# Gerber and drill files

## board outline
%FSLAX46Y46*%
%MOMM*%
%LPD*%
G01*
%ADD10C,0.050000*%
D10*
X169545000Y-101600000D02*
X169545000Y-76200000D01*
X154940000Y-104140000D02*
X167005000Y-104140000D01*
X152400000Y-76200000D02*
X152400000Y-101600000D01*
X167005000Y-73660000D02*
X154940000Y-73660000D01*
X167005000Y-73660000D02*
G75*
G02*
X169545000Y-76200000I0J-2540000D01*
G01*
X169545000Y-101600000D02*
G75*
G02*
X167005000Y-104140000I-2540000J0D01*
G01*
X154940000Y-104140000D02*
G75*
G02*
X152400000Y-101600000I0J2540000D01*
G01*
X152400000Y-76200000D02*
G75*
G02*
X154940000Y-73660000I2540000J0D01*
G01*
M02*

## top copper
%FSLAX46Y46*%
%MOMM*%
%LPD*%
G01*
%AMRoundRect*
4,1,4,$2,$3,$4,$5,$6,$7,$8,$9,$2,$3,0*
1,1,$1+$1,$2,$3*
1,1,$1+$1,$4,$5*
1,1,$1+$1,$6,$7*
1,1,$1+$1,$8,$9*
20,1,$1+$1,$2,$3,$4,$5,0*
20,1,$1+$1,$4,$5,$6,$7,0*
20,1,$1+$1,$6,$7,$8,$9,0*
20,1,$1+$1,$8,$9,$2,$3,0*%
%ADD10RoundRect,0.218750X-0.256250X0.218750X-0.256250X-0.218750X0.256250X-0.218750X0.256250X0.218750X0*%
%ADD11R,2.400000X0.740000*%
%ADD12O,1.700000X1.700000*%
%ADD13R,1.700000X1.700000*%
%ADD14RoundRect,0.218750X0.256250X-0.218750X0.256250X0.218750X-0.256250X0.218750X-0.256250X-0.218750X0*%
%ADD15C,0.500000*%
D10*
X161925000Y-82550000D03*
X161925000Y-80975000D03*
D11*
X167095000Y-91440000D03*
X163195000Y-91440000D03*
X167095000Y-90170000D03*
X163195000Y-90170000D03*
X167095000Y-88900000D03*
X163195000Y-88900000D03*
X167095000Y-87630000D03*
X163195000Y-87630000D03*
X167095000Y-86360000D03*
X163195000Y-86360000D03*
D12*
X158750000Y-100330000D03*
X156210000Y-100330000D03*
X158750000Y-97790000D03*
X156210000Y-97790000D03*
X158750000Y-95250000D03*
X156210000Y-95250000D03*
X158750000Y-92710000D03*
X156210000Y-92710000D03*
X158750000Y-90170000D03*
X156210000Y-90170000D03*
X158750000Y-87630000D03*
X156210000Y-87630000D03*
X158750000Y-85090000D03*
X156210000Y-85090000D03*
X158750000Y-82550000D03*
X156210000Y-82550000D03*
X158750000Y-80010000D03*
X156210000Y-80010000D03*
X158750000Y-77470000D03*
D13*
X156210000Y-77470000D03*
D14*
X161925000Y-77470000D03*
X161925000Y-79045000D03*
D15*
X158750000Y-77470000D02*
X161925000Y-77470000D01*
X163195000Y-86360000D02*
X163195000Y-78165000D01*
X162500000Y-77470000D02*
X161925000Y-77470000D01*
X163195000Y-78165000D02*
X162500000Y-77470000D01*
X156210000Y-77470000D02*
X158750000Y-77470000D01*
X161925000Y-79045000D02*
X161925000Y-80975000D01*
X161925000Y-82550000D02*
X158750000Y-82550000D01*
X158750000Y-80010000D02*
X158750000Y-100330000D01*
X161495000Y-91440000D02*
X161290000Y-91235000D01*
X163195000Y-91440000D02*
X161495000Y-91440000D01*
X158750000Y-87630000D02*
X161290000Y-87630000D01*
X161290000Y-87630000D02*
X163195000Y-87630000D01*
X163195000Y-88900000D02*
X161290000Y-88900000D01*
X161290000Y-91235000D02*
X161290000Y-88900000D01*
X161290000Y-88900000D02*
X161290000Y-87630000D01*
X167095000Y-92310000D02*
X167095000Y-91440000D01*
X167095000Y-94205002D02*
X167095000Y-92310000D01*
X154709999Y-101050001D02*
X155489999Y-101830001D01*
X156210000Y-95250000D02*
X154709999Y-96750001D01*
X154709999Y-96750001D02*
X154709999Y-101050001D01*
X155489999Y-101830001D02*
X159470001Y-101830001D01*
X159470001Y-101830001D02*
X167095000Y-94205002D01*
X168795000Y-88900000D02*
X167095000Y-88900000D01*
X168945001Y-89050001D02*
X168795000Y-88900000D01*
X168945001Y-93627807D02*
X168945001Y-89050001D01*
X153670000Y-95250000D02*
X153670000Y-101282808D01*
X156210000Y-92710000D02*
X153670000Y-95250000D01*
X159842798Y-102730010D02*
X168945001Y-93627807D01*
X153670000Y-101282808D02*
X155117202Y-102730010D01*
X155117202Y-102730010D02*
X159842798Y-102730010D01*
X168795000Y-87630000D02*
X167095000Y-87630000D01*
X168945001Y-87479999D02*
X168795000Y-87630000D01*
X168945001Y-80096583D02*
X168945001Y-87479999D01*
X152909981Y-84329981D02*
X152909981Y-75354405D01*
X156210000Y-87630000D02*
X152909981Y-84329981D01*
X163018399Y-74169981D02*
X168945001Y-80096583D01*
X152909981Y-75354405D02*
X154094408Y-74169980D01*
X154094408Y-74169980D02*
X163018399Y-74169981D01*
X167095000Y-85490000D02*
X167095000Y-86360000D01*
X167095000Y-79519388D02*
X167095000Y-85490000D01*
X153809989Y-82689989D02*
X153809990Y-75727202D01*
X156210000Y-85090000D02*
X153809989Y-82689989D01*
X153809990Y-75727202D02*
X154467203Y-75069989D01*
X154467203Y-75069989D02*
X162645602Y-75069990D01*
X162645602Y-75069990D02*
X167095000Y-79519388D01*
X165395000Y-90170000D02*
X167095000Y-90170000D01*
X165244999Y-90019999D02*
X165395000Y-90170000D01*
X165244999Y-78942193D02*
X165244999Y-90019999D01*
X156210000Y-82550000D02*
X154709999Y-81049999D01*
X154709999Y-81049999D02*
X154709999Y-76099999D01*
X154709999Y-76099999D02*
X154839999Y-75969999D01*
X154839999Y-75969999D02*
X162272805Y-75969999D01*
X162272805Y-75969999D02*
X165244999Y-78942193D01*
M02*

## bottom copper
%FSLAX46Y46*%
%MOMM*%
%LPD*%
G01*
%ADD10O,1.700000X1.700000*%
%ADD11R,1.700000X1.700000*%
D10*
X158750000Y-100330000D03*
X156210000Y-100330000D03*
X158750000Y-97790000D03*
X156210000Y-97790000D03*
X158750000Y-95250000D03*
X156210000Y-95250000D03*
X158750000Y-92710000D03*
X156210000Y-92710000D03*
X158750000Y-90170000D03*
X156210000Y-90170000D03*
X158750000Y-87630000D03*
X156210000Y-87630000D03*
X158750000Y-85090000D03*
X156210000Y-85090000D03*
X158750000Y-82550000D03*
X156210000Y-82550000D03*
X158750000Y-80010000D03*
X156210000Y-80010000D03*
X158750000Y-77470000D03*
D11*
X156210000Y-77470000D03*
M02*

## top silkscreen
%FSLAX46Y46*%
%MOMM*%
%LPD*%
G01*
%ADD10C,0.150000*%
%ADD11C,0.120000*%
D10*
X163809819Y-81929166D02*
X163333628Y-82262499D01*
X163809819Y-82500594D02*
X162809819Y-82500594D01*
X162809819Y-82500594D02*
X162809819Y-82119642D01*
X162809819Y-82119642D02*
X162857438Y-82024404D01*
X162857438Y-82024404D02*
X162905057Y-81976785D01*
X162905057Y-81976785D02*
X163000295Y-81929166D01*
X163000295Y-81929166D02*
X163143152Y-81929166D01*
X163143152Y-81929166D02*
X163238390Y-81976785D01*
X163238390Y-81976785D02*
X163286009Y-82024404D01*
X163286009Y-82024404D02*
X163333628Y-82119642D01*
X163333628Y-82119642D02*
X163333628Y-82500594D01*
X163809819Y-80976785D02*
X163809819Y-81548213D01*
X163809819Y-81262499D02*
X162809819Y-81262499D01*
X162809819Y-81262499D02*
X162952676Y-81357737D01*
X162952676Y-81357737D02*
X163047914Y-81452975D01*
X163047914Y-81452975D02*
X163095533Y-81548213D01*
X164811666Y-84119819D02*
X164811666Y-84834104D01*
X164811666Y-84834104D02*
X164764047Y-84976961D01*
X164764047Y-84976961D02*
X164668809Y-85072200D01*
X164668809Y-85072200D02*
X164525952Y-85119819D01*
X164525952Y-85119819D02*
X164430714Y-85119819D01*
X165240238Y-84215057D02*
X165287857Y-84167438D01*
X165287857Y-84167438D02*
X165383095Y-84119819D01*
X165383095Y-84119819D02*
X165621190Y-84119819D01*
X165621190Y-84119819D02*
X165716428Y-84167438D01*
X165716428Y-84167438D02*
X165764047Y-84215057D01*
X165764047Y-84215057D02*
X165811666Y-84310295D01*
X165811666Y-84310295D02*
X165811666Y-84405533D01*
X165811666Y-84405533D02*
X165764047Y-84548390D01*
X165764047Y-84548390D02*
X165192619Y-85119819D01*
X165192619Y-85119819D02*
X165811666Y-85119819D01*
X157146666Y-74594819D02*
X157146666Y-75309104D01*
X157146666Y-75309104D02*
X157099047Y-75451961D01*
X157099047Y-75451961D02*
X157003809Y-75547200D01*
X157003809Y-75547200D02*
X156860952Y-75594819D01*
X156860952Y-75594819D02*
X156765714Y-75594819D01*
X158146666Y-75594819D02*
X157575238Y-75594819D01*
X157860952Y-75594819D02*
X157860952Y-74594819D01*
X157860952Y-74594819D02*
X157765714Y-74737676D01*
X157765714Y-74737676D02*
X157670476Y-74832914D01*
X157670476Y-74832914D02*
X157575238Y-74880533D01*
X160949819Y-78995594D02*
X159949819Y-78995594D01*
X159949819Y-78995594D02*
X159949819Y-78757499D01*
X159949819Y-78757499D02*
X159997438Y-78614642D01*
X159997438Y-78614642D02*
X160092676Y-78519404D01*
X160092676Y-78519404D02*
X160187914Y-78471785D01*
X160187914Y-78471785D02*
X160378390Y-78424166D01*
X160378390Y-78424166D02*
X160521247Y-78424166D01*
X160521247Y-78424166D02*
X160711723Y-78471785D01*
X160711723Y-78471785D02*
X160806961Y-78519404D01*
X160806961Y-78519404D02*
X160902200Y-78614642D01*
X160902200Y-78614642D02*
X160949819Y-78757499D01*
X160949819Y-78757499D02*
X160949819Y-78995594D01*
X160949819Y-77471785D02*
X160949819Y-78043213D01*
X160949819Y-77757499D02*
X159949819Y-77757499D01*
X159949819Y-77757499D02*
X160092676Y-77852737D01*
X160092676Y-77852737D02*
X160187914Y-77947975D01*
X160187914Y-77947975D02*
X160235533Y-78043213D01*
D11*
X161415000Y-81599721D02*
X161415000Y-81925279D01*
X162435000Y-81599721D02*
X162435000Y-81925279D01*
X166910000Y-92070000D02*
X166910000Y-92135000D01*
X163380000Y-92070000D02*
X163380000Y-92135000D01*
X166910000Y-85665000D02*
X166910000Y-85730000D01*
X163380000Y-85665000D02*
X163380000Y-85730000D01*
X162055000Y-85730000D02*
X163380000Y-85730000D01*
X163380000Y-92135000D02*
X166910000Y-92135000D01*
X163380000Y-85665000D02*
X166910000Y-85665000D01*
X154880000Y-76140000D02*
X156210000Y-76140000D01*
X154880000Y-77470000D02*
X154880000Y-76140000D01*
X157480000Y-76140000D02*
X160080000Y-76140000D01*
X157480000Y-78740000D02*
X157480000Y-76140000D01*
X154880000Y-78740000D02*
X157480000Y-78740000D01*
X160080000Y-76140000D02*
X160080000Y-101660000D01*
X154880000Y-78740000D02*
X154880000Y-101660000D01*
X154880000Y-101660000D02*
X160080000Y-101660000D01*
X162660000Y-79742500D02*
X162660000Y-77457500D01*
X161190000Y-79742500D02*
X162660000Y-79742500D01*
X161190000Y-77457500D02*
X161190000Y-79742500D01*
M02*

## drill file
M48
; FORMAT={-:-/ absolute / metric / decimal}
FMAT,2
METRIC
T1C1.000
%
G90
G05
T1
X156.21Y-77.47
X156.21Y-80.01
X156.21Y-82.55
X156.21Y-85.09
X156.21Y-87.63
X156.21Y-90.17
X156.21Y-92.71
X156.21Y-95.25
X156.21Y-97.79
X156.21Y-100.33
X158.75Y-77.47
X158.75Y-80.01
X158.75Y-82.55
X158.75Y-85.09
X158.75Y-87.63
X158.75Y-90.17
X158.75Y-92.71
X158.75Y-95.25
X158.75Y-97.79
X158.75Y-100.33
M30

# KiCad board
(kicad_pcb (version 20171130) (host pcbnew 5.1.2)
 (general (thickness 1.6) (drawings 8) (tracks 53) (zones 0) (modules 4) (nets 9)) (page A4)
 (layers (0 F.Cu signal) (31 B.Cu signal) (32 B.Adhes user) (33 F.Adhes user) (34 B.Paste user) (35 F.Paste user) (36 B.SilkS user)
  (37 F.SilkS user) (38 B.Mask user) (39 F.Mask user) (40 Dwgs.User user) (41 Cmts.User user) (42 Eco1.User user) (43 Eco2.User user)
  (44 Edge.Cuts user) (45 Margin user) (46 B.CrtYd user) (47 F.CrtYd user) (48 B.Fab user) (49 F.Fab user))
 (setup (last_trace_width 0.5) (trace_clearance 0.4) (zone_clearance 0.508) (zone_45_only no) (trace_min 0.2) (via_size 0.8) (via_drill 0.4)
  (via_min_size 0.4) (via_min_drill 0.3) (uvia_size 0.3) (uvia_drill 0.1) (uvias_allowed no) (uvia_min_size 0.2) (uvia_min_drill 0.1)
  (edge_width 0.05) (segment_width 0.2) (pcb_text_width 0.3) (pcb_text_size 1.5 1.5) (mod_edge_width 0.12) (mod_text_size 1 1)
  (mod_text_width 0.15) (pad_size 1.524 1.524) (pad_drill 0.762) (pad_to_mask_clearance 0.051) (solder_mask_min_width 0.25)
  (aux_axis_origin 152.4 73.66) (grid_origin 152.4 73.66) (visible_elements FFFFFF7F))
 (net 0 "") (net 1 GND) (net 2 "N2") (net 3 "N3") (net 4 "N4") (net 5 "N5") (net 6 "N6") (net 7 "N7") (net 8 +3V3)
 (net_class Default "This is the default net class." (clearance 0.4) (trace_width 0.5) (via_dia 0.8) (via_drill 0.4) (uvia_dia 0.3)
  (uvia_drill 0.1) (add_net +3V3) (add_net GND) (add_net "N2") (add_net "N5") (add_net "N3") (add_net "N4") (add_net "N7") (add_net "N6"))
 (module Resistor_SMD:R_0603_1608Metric (layer F.Cu) (at 161.925 81.7625 270)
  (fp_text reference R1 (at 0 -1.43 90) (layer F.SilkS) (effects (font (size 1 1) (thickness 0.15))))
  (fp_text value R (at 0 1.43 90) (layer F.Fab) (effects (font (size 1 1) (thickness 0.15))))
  (fp_line (start -0.162779 0.51) (end 0.162779 0.51) (layer F.SilkS) (width 0.12))
  (fp_line (start -0.162779 -0.51) (end 0.162779 -0.51) (layer F.SilkS) (width 0.12))
  (pad 2 smd roundrect (at 0.7875 0 270) (size 0.875 0.95) (layers F.Cu F.Paste F.Mask) (roundrect_rratio 0.25) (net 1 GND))
  (pad 1 smd roundrect (at -0.7875 0 270) (size 0.875 0.95) (layers F.Cu F.Paste F.Mask) (roundrect_rratio 0.25) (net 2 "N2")))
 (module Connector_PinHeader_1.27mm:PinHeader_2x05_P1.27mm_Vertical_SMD (layer F.Cu) (at 165.145 88.9)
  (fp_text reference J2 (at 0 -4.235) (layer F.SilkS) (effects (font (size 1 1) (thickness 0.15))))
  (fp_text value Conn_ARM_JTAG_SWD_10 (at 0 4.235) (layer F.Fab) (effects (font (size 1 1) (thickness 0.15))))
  (fp_line (start 1.765 3.17) (end 1.765 3.235) (layer F.SilkS) (width 0.12))
  (fp_line (start -1.765 3.17) (end -1.765 3.235) (layer F.SilkS) (width 0.12))
  (fp_line (start 1.765 -3.235) (end 1.765 -3.17) (layer F.SilkS) (width 0.12))
  (fp_line (start -1.765 -3.235) (end -1.765 -3.17) (layer F.SilkS) (width 0.12))
  (fp_line (start -3.09 -3.17) (end -1.765 -3.17) (layer F.SilkS) (width 0.12))
  (fp_line (start -1.765 3.235) (end 1.765 3.235) (layer F.SilkS) (width 0.12))
  (fp_line (start -1.765 -3.235) (end 1.765 -3.235) (layer F.SilkS) (width 0.12))
  (pad 10 smd rect (at 1.95 2.54) (size 2.4 0.74) (layers F.Cu F.Paste F.Mask) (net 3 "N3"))
  (pad 9 smd rect (at -1.95 2.54) (size 2.4 0.74) (layers F.Cu F.Paste F.Mask) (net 1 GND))
  (pad 8 smd rect (at 1.95 1.27) (size 2.4 0.74) (layers F.Cu F.Paste F.Mask) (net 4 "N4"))
  (pad 7 smd rect (at -1.95 1.27) (size 2.4 0.74) (layers F.Cu F.Paste F.Mask))
  (pad 6 smd rect (at 1.95 0) (size 2.4 0.74) (layers F.Cu F.Paste F.Mask) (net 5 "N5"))
  (pad 5 smd rect (at -1.95 0) (size 2.4 0.74) (layers F.Cu F.Paste F.Mask) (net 1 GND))
  (pad 4 smd rect (at 1.95 -1.27) (size 2.4 0.74) (layers F.Cu F.Paste F.Mask) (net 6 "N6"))
  (pad 3 smd rect (at -1.95 -1.27) (size 2.4 0.74) (layers F.Cu F.Paste F.Mask) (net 1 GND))
  (pad 2 smd rect (at 1.95 -2.54) (size 2.4 0.74) (layers F.Cu F.Paste F.Mask) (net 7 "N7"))
  (pad 1 smd rect (at -1.95 -2.54) (size 2.4 0.74) (layers F.Cu F.Paste F.Mask) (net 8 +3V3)))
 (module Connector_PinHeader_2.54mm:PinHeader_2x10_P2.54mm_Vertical (layer F.Cu) (at 156.21 77.47)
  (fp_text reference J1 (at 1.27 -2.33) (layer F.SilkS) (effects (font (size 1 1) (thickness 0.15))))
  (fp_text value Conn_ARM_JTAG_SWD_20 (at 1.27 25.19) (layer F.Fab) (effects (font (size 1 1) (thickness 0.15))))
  (fp_line (start -1.33 -1.33) (end 0 -1.33) (layer F.SilkS) (width 0.12))
  (fp_line (start -1.33 0) (end -1.33 -1.33) (layer F.SilkS) (width 0.12))
  (fp_line (start 1.27 -1.33) (end 3.87 -1.33) (layer F.SilkS) (width 0.12))
  (fp_line (start 1.27 1.27) (end 1.27 -1.33) (layer F.SilkS) (width 0.12))
  (fp_line (start -1.33 1.27) (end 1.27 1.27) (layer F.SilkS) (width 0.12))
  (fp_line (start 3.87 -1.33) (end 3.87 24.19) (layer F.SilkS) (width 0.12))
  (fp_line (start -1.33 1.27) (end -1.33 24.19) (layer F.SilkS) (width 0.12))
  (fp_line (start -1.33 24.19) (end 3.87 24.19) (layer F.SilkS) (width 0.12))
  (pad 20 thru_hole oval (at 2.54 22.86) (size 1.7 1.7) (drill 1) (layers *.Cu *.Mask) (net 1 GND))
  (pad 19 thru_hole oval (at 0 22.86) (size 1.7 1.7) (drill 1) (layers *.Cu *.Mask))
  (pad 18 thru_hole oval (at 2.54 20.32) (size 1.7 1.7) (drill 1) (layers *.Cu *.Mask) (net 1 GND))
  (pad 17 thru_hole oval (at 0 20.32) (size 1.7 1.7) (drill 1) (layers *.Cu *.Mask))
  (pad 16 thru_hole oval (at 2.54 17.78) (size 1.7 1.7) (drill 1) (layers *.Cu *.Mask) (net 1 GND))
  (pad 15 thru_hole oval (at 0 17.78) (size 1.7 1.7) (drill 1) (layers *.Cu *.Mask) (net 3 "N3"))
  (pad 14 thru_hole oval (at 2.54 15.24) (size 1.7 1.7) (drill 1) (layers *.Cu *.Mask) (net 1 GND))
  (pad 13 thru_hole oval (at 0 15.24) (size 1.7 1.7) (drill 1) (layers *.Cu *.Mask) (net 5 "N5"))
  (pad 12 thru_hole oval (at 2.54 12.7) (size 1.7 1.7) (drill 1) (layers *.Cu *.Mask) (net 1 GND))
  (pad 11 thru_hole oval (at 0 12.7) (size 1.7 1.7) (drill 1) (layers *.Cu *.Mask))
  (pad 10 thru_hole oval (at 2.54 10.16) (size 1.7 1.7) (drill 1) (layers *.Cu *.Mask) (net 1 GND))
  (pad 9 thru_hole oval (at 0 10.16) (size 1.7 1.7) (drill 1) (layers *.Cu *.Mask) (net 6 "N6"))
  (pad 8 thru_hole oval (at 2.54 7.62) (size 1.7 1.7) (drill 1) (layers *.Cu *.Mask) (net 1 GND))
  (pad 7 thru_hole oval (at 0 7.62) (size 1.7 1.7) (drill 1) (layers *.Cu *.Mask) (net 7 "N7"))
  (pad 6 thru_hole oval (at 2.54 5.08) (size 1.7 1.7) (drill 1) (layers *.Cu *.Mask) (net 1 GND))
  (pad 5 thru_hole oval (at 0 5.08) (size 1.7 1.7) (drill 1) (layers *.Cu *.Mask) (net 4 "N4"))
  (pad 4 thru_hole oval (at 2.54 2.54) (size 1.7 1.7) (drill 1) (layers *.Cu *.Mask) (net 1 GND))
  (pad 3 thru_hole oval (at 0 2.54) (size 1.7 1.7) (drill 1) (layers *.Cu *.Mask))
  (pad 2 thru_hole oval (at 2.54 0) (size 1.7 1.7) (drill 1) (layers *.Cu *.Mask) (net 8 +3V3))
  (pad 1 thru_hole rect (at 0 0) (size 1.7 1.7) (drill 1) (layers *.Cu *.Mask) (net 8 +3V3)))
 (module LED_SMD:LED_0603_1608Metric (layer F.Cu) (at 161.925 78.2575 90)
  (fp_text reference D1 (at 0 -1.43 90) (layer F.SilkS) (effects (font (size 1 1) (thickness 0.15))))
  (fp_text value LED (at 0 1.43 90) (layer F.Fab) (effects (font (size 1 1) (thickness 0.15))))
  (fp_line (start -1.485 0.735) (end 0.8 0.735) (layer F.SilkS) (width 0.12))
  (fp_line (start -1.485 -0.735) (end -1.485 0.735) (layer F.SilkS) (width 0.12))
  (fp_line (start 0.8 -0.735) (end -1.485 -0.735) (layer F.SilkS) (width 0.12))
  (pad 2 smd roundrect (at 0.7875 0 90) (size 0.875 0.95) (layers F.Cu F.Paste F.Mask) (roundrect_rratio 0.25) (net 8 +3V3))
  (pad 1 smd roundrect (at -0.7875 0 90) (size 0.875 0.95) (layers F.Cu F.Paste F.Mask) (roundrect_rratio 0.25) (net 2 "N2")))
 (gr_line (start 169.545 101.6) (end 169.545 76.2) (layer Edge.Cuts) (width 0.05))
 (gr_line (start 154.94 104.14) (end 167.005 104.14) (layer Edge.Cuts) (width 0.05))
 (gr_line (start 152.4 76.2) (end 152.4 101.6) (layer Edge.Cuts) (width 0.05))
 (gr_line (start 167.005 73.66) (end 154.94 73.66) (layer Edge.Cuts) (width 0.05))
 (gr_arc (start 167.005 76.2) (end 169.545 76.2) (angle -90) (layer Edge.Cuts) (width 0.05))
 (gr_arc (start 167.005 101.6) (end 167.005 104.14) (angle -90) (layer Edge.Cuts) (width 0.05))
 (gr_arc (start 154.94 101.6) (end 152.4 101.6) (angle -90) (layer Edge.Cuts) (width 0.05))
 (gr_arc (start 154.94 76.2) (end 154.94 73.66) (angle -90) (layer Edge.Cuts) (width 0.05))
 (segment (start 158.75 77.47) (end 161.925 77.47) (width 0.5) (layer F.Cu) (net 8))
 (segment (start 163.195 86.36) (end 163.195 78.165) (width 0.5) (layer F.Cu) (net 8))
 (segment (start 162.5 77.47) (end 161.925 77.47) (width 0.5) (layer F.Cu) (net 8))
 (segment (start 163.195 78.165) (end 162.5 77.47) (width 0.5) (layer F.Cu) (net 8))
 (segment (start 156.21 77.47) (end 158.75 77.47) (width 0.5) (layer F.Cu) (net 8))
 (segment (start 161.925 79.045) (end 161.925 80.975) (width 0.5) (layer F.Cu) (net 2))
 (segment (start 161.925 82.55) (end 158.75 82.55) (width 0.5) (layer F.Cu) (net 1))
 (segment (start 158.75 80.01) (end 158.75 100.33) (width 0.5) (layer F.Cu) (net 1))
 (segment (start 161.495 91.44) (end 161.29 91.235) (width 0.5) (layer F.Cu) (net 1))
 (segment (start 163.195 91.44) (end 161.495 91.44) (width 0.5) (layer F.Cu) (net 1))
 (segment (start 158.75 87.63) (end 161.29 87.63) (width 0.5) (layer F.Cu) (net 1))
 (segment (start 161.29 87.63) (end 163.195 87.63) (width 0.5) (layer F.Cu) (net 1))
 (segment (start 163.195 88.9) (end 161.29 88.9) (width 0.5) (layer F.Cu) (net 1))
 (segment (start 161.29 91.235) (end 161.29 88.9) (width 0.5) (layer F.Cu) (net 1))
 (segment (start 161.29 88.9) (end 161.29 87.63) (width 0.5) (layer F.Cu) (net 1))
 (segment (start 167.095 92.31) (end 167.095 91.44) (width 0.5) (layer F.Cu) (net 3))
 (segment (start 167.095 94.205002) (end 167.095 92.31) (width 0.5) (layer F.Cu) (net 3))
 (segment (start 154.709999 101.050001) (end 155.489999 101.830001) (width 0.5) (layer F.Cu) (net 3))
 (segment (start 156.21 95.25) (end 154.709999 96.750001) (width 0.5) (layer F.Cu) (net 3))
 (segment (start 154.709999 96.750001) (end 154.709999 101.050001) (width 0.5) (layer F.Cu) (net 3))
 (segment (start 155.489999 101.830001) (end 159.470001 101.830001) (width 0.5) (layer F.Cu) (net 3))
 (segment (start 159.470001 101.830001) (end 167.095 94.205002) (width 0.5) (layer F.Cu) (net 3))
 (segment (start 168.795 88.9) (end 167.095 88.9) (width 0.5) (layer F.Cu) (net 5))
 (segment (start 168.945001 89.050001) (end 168.795 88.9) (width 0.5) (layer F.Cu) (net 5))
 (segment (start 168.945001 93.627807) (end 168.945001 89.050001) (width 0.5) (layer F.Cu) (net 5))
 (segment (start 153.67 95.25) (end 153.67 101.282808) (width 0.5) (layer F.Cu) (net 5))
 (segment (start 156.21 92.71) (end 153.67 95.25) (width 0.5) (layer F.Cu) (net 5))
 (segment (start 159.842798 102.73001) (end 168.945001 93.627807) (width 0.5) (layer F.Cu) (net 5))
 (segment (start 153.67 101.282808) (end 155.117202 102.73001) (width 0.5) (layer F.Cu) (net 5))
 (segment (start 155.117202 102.73001) (end 159.842798 102.73001) (width 0.5) (layer F.Cu) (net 5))
 (segment (start 168.795 87.63) (end 167.095 87.63) (width 0.5) (layer F.Cu) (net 6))
 (segment (start 168.945001 87.479999) (end 168.795 87.63) (width 0.5) (layer F.Cu) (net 6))
 (segment (start 168.945001 80.096583) (end 168.945001 87.479999) (width 0.5) (layer F.Cu) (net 6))
 (segment (start 152.909981 84.329981) (end 152.909981 75.354405) (width 0.5) (layer F.Cu) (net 6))
 (segment (start 156.21 87.63) (end 152.909981 84.329981) (width 0.5) (layer F.Cu) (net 6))
 (segment (start 163.018399 74.169981) (end 168.945001 80.096583) (width 0.5) (layer F.Cu) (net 6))
 (segment (start 152.909981 75.354405) (end 154.094408 74.16998) (width 0.5) (layer F.Cu) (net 6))
 (segment (start 154.094408 74.16998) (end 163.018399 74.169981) (width 0.5) (layer F.Cu) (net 6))
 (segment (start 167.095 85.49) (end 167.095 86.36) (width 0.5) (layer F.Cu) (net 7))
 (segment (start 167.095 79.519388) (end 167.095 85.49) (width 0.5) (layer F.Cu) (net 7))
 (segment (start 153.809989 82.689989) (end 153.80999 75.727202) (width 0.5) (layer F.Cu) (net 7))
 (segment (start 156.21 85.09) (end 153.809989 82.689989) (width 0.5) (layer F.Cu) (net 7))
 (segment (start 153.80999 75.727202) (end 154.467203 75.069989) (width 0.5) (layer F.Cu) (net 7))
 (segment (start 154.467203 75.069989) (end 162.645602 75.06999) (width 0.5) (layer F.Cu) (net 7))
 (segment (start 162.645602 75.06999) (end 167.095 79.519388) (width 0.5) (layer F.Cu) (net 7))
 (segment (start 165.395 90.17) (end 167.095 90.17) (width 0.5) (layer F.Cu) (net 4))
 (segment (start 165.244999 90.019999) (end 165.395 90.17) (width 0.5) (layer F.Cu) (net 4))
 (segment (start 165.244999 78.942193) (end 165.244999 90.019999) (width 0.5) (layer F.Cu) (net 4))
 (segment (start 156.21 82.55) (end 154.709999 81.049999) (width 0.5) (layer F.Cu) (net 4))
 (segment (start 154.709999 81.049999) (end 154.709999 76.099999) (width 0.5) (layer F.Cu) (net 4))
 (segment (start 154.709999 76.099999) (end 154.839999 75.969999) (width 0.5) (layer F.Cu) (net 4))
 (segment (start 154.839999 75.969999) (end 162.272805 75.969999) (width 0.5) (layer F.Cu) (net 4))
 (segment (start 162.272805 75.969999) (end 165.244999 78.942193) (width 0.5) (layer F.Cu) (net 4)))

